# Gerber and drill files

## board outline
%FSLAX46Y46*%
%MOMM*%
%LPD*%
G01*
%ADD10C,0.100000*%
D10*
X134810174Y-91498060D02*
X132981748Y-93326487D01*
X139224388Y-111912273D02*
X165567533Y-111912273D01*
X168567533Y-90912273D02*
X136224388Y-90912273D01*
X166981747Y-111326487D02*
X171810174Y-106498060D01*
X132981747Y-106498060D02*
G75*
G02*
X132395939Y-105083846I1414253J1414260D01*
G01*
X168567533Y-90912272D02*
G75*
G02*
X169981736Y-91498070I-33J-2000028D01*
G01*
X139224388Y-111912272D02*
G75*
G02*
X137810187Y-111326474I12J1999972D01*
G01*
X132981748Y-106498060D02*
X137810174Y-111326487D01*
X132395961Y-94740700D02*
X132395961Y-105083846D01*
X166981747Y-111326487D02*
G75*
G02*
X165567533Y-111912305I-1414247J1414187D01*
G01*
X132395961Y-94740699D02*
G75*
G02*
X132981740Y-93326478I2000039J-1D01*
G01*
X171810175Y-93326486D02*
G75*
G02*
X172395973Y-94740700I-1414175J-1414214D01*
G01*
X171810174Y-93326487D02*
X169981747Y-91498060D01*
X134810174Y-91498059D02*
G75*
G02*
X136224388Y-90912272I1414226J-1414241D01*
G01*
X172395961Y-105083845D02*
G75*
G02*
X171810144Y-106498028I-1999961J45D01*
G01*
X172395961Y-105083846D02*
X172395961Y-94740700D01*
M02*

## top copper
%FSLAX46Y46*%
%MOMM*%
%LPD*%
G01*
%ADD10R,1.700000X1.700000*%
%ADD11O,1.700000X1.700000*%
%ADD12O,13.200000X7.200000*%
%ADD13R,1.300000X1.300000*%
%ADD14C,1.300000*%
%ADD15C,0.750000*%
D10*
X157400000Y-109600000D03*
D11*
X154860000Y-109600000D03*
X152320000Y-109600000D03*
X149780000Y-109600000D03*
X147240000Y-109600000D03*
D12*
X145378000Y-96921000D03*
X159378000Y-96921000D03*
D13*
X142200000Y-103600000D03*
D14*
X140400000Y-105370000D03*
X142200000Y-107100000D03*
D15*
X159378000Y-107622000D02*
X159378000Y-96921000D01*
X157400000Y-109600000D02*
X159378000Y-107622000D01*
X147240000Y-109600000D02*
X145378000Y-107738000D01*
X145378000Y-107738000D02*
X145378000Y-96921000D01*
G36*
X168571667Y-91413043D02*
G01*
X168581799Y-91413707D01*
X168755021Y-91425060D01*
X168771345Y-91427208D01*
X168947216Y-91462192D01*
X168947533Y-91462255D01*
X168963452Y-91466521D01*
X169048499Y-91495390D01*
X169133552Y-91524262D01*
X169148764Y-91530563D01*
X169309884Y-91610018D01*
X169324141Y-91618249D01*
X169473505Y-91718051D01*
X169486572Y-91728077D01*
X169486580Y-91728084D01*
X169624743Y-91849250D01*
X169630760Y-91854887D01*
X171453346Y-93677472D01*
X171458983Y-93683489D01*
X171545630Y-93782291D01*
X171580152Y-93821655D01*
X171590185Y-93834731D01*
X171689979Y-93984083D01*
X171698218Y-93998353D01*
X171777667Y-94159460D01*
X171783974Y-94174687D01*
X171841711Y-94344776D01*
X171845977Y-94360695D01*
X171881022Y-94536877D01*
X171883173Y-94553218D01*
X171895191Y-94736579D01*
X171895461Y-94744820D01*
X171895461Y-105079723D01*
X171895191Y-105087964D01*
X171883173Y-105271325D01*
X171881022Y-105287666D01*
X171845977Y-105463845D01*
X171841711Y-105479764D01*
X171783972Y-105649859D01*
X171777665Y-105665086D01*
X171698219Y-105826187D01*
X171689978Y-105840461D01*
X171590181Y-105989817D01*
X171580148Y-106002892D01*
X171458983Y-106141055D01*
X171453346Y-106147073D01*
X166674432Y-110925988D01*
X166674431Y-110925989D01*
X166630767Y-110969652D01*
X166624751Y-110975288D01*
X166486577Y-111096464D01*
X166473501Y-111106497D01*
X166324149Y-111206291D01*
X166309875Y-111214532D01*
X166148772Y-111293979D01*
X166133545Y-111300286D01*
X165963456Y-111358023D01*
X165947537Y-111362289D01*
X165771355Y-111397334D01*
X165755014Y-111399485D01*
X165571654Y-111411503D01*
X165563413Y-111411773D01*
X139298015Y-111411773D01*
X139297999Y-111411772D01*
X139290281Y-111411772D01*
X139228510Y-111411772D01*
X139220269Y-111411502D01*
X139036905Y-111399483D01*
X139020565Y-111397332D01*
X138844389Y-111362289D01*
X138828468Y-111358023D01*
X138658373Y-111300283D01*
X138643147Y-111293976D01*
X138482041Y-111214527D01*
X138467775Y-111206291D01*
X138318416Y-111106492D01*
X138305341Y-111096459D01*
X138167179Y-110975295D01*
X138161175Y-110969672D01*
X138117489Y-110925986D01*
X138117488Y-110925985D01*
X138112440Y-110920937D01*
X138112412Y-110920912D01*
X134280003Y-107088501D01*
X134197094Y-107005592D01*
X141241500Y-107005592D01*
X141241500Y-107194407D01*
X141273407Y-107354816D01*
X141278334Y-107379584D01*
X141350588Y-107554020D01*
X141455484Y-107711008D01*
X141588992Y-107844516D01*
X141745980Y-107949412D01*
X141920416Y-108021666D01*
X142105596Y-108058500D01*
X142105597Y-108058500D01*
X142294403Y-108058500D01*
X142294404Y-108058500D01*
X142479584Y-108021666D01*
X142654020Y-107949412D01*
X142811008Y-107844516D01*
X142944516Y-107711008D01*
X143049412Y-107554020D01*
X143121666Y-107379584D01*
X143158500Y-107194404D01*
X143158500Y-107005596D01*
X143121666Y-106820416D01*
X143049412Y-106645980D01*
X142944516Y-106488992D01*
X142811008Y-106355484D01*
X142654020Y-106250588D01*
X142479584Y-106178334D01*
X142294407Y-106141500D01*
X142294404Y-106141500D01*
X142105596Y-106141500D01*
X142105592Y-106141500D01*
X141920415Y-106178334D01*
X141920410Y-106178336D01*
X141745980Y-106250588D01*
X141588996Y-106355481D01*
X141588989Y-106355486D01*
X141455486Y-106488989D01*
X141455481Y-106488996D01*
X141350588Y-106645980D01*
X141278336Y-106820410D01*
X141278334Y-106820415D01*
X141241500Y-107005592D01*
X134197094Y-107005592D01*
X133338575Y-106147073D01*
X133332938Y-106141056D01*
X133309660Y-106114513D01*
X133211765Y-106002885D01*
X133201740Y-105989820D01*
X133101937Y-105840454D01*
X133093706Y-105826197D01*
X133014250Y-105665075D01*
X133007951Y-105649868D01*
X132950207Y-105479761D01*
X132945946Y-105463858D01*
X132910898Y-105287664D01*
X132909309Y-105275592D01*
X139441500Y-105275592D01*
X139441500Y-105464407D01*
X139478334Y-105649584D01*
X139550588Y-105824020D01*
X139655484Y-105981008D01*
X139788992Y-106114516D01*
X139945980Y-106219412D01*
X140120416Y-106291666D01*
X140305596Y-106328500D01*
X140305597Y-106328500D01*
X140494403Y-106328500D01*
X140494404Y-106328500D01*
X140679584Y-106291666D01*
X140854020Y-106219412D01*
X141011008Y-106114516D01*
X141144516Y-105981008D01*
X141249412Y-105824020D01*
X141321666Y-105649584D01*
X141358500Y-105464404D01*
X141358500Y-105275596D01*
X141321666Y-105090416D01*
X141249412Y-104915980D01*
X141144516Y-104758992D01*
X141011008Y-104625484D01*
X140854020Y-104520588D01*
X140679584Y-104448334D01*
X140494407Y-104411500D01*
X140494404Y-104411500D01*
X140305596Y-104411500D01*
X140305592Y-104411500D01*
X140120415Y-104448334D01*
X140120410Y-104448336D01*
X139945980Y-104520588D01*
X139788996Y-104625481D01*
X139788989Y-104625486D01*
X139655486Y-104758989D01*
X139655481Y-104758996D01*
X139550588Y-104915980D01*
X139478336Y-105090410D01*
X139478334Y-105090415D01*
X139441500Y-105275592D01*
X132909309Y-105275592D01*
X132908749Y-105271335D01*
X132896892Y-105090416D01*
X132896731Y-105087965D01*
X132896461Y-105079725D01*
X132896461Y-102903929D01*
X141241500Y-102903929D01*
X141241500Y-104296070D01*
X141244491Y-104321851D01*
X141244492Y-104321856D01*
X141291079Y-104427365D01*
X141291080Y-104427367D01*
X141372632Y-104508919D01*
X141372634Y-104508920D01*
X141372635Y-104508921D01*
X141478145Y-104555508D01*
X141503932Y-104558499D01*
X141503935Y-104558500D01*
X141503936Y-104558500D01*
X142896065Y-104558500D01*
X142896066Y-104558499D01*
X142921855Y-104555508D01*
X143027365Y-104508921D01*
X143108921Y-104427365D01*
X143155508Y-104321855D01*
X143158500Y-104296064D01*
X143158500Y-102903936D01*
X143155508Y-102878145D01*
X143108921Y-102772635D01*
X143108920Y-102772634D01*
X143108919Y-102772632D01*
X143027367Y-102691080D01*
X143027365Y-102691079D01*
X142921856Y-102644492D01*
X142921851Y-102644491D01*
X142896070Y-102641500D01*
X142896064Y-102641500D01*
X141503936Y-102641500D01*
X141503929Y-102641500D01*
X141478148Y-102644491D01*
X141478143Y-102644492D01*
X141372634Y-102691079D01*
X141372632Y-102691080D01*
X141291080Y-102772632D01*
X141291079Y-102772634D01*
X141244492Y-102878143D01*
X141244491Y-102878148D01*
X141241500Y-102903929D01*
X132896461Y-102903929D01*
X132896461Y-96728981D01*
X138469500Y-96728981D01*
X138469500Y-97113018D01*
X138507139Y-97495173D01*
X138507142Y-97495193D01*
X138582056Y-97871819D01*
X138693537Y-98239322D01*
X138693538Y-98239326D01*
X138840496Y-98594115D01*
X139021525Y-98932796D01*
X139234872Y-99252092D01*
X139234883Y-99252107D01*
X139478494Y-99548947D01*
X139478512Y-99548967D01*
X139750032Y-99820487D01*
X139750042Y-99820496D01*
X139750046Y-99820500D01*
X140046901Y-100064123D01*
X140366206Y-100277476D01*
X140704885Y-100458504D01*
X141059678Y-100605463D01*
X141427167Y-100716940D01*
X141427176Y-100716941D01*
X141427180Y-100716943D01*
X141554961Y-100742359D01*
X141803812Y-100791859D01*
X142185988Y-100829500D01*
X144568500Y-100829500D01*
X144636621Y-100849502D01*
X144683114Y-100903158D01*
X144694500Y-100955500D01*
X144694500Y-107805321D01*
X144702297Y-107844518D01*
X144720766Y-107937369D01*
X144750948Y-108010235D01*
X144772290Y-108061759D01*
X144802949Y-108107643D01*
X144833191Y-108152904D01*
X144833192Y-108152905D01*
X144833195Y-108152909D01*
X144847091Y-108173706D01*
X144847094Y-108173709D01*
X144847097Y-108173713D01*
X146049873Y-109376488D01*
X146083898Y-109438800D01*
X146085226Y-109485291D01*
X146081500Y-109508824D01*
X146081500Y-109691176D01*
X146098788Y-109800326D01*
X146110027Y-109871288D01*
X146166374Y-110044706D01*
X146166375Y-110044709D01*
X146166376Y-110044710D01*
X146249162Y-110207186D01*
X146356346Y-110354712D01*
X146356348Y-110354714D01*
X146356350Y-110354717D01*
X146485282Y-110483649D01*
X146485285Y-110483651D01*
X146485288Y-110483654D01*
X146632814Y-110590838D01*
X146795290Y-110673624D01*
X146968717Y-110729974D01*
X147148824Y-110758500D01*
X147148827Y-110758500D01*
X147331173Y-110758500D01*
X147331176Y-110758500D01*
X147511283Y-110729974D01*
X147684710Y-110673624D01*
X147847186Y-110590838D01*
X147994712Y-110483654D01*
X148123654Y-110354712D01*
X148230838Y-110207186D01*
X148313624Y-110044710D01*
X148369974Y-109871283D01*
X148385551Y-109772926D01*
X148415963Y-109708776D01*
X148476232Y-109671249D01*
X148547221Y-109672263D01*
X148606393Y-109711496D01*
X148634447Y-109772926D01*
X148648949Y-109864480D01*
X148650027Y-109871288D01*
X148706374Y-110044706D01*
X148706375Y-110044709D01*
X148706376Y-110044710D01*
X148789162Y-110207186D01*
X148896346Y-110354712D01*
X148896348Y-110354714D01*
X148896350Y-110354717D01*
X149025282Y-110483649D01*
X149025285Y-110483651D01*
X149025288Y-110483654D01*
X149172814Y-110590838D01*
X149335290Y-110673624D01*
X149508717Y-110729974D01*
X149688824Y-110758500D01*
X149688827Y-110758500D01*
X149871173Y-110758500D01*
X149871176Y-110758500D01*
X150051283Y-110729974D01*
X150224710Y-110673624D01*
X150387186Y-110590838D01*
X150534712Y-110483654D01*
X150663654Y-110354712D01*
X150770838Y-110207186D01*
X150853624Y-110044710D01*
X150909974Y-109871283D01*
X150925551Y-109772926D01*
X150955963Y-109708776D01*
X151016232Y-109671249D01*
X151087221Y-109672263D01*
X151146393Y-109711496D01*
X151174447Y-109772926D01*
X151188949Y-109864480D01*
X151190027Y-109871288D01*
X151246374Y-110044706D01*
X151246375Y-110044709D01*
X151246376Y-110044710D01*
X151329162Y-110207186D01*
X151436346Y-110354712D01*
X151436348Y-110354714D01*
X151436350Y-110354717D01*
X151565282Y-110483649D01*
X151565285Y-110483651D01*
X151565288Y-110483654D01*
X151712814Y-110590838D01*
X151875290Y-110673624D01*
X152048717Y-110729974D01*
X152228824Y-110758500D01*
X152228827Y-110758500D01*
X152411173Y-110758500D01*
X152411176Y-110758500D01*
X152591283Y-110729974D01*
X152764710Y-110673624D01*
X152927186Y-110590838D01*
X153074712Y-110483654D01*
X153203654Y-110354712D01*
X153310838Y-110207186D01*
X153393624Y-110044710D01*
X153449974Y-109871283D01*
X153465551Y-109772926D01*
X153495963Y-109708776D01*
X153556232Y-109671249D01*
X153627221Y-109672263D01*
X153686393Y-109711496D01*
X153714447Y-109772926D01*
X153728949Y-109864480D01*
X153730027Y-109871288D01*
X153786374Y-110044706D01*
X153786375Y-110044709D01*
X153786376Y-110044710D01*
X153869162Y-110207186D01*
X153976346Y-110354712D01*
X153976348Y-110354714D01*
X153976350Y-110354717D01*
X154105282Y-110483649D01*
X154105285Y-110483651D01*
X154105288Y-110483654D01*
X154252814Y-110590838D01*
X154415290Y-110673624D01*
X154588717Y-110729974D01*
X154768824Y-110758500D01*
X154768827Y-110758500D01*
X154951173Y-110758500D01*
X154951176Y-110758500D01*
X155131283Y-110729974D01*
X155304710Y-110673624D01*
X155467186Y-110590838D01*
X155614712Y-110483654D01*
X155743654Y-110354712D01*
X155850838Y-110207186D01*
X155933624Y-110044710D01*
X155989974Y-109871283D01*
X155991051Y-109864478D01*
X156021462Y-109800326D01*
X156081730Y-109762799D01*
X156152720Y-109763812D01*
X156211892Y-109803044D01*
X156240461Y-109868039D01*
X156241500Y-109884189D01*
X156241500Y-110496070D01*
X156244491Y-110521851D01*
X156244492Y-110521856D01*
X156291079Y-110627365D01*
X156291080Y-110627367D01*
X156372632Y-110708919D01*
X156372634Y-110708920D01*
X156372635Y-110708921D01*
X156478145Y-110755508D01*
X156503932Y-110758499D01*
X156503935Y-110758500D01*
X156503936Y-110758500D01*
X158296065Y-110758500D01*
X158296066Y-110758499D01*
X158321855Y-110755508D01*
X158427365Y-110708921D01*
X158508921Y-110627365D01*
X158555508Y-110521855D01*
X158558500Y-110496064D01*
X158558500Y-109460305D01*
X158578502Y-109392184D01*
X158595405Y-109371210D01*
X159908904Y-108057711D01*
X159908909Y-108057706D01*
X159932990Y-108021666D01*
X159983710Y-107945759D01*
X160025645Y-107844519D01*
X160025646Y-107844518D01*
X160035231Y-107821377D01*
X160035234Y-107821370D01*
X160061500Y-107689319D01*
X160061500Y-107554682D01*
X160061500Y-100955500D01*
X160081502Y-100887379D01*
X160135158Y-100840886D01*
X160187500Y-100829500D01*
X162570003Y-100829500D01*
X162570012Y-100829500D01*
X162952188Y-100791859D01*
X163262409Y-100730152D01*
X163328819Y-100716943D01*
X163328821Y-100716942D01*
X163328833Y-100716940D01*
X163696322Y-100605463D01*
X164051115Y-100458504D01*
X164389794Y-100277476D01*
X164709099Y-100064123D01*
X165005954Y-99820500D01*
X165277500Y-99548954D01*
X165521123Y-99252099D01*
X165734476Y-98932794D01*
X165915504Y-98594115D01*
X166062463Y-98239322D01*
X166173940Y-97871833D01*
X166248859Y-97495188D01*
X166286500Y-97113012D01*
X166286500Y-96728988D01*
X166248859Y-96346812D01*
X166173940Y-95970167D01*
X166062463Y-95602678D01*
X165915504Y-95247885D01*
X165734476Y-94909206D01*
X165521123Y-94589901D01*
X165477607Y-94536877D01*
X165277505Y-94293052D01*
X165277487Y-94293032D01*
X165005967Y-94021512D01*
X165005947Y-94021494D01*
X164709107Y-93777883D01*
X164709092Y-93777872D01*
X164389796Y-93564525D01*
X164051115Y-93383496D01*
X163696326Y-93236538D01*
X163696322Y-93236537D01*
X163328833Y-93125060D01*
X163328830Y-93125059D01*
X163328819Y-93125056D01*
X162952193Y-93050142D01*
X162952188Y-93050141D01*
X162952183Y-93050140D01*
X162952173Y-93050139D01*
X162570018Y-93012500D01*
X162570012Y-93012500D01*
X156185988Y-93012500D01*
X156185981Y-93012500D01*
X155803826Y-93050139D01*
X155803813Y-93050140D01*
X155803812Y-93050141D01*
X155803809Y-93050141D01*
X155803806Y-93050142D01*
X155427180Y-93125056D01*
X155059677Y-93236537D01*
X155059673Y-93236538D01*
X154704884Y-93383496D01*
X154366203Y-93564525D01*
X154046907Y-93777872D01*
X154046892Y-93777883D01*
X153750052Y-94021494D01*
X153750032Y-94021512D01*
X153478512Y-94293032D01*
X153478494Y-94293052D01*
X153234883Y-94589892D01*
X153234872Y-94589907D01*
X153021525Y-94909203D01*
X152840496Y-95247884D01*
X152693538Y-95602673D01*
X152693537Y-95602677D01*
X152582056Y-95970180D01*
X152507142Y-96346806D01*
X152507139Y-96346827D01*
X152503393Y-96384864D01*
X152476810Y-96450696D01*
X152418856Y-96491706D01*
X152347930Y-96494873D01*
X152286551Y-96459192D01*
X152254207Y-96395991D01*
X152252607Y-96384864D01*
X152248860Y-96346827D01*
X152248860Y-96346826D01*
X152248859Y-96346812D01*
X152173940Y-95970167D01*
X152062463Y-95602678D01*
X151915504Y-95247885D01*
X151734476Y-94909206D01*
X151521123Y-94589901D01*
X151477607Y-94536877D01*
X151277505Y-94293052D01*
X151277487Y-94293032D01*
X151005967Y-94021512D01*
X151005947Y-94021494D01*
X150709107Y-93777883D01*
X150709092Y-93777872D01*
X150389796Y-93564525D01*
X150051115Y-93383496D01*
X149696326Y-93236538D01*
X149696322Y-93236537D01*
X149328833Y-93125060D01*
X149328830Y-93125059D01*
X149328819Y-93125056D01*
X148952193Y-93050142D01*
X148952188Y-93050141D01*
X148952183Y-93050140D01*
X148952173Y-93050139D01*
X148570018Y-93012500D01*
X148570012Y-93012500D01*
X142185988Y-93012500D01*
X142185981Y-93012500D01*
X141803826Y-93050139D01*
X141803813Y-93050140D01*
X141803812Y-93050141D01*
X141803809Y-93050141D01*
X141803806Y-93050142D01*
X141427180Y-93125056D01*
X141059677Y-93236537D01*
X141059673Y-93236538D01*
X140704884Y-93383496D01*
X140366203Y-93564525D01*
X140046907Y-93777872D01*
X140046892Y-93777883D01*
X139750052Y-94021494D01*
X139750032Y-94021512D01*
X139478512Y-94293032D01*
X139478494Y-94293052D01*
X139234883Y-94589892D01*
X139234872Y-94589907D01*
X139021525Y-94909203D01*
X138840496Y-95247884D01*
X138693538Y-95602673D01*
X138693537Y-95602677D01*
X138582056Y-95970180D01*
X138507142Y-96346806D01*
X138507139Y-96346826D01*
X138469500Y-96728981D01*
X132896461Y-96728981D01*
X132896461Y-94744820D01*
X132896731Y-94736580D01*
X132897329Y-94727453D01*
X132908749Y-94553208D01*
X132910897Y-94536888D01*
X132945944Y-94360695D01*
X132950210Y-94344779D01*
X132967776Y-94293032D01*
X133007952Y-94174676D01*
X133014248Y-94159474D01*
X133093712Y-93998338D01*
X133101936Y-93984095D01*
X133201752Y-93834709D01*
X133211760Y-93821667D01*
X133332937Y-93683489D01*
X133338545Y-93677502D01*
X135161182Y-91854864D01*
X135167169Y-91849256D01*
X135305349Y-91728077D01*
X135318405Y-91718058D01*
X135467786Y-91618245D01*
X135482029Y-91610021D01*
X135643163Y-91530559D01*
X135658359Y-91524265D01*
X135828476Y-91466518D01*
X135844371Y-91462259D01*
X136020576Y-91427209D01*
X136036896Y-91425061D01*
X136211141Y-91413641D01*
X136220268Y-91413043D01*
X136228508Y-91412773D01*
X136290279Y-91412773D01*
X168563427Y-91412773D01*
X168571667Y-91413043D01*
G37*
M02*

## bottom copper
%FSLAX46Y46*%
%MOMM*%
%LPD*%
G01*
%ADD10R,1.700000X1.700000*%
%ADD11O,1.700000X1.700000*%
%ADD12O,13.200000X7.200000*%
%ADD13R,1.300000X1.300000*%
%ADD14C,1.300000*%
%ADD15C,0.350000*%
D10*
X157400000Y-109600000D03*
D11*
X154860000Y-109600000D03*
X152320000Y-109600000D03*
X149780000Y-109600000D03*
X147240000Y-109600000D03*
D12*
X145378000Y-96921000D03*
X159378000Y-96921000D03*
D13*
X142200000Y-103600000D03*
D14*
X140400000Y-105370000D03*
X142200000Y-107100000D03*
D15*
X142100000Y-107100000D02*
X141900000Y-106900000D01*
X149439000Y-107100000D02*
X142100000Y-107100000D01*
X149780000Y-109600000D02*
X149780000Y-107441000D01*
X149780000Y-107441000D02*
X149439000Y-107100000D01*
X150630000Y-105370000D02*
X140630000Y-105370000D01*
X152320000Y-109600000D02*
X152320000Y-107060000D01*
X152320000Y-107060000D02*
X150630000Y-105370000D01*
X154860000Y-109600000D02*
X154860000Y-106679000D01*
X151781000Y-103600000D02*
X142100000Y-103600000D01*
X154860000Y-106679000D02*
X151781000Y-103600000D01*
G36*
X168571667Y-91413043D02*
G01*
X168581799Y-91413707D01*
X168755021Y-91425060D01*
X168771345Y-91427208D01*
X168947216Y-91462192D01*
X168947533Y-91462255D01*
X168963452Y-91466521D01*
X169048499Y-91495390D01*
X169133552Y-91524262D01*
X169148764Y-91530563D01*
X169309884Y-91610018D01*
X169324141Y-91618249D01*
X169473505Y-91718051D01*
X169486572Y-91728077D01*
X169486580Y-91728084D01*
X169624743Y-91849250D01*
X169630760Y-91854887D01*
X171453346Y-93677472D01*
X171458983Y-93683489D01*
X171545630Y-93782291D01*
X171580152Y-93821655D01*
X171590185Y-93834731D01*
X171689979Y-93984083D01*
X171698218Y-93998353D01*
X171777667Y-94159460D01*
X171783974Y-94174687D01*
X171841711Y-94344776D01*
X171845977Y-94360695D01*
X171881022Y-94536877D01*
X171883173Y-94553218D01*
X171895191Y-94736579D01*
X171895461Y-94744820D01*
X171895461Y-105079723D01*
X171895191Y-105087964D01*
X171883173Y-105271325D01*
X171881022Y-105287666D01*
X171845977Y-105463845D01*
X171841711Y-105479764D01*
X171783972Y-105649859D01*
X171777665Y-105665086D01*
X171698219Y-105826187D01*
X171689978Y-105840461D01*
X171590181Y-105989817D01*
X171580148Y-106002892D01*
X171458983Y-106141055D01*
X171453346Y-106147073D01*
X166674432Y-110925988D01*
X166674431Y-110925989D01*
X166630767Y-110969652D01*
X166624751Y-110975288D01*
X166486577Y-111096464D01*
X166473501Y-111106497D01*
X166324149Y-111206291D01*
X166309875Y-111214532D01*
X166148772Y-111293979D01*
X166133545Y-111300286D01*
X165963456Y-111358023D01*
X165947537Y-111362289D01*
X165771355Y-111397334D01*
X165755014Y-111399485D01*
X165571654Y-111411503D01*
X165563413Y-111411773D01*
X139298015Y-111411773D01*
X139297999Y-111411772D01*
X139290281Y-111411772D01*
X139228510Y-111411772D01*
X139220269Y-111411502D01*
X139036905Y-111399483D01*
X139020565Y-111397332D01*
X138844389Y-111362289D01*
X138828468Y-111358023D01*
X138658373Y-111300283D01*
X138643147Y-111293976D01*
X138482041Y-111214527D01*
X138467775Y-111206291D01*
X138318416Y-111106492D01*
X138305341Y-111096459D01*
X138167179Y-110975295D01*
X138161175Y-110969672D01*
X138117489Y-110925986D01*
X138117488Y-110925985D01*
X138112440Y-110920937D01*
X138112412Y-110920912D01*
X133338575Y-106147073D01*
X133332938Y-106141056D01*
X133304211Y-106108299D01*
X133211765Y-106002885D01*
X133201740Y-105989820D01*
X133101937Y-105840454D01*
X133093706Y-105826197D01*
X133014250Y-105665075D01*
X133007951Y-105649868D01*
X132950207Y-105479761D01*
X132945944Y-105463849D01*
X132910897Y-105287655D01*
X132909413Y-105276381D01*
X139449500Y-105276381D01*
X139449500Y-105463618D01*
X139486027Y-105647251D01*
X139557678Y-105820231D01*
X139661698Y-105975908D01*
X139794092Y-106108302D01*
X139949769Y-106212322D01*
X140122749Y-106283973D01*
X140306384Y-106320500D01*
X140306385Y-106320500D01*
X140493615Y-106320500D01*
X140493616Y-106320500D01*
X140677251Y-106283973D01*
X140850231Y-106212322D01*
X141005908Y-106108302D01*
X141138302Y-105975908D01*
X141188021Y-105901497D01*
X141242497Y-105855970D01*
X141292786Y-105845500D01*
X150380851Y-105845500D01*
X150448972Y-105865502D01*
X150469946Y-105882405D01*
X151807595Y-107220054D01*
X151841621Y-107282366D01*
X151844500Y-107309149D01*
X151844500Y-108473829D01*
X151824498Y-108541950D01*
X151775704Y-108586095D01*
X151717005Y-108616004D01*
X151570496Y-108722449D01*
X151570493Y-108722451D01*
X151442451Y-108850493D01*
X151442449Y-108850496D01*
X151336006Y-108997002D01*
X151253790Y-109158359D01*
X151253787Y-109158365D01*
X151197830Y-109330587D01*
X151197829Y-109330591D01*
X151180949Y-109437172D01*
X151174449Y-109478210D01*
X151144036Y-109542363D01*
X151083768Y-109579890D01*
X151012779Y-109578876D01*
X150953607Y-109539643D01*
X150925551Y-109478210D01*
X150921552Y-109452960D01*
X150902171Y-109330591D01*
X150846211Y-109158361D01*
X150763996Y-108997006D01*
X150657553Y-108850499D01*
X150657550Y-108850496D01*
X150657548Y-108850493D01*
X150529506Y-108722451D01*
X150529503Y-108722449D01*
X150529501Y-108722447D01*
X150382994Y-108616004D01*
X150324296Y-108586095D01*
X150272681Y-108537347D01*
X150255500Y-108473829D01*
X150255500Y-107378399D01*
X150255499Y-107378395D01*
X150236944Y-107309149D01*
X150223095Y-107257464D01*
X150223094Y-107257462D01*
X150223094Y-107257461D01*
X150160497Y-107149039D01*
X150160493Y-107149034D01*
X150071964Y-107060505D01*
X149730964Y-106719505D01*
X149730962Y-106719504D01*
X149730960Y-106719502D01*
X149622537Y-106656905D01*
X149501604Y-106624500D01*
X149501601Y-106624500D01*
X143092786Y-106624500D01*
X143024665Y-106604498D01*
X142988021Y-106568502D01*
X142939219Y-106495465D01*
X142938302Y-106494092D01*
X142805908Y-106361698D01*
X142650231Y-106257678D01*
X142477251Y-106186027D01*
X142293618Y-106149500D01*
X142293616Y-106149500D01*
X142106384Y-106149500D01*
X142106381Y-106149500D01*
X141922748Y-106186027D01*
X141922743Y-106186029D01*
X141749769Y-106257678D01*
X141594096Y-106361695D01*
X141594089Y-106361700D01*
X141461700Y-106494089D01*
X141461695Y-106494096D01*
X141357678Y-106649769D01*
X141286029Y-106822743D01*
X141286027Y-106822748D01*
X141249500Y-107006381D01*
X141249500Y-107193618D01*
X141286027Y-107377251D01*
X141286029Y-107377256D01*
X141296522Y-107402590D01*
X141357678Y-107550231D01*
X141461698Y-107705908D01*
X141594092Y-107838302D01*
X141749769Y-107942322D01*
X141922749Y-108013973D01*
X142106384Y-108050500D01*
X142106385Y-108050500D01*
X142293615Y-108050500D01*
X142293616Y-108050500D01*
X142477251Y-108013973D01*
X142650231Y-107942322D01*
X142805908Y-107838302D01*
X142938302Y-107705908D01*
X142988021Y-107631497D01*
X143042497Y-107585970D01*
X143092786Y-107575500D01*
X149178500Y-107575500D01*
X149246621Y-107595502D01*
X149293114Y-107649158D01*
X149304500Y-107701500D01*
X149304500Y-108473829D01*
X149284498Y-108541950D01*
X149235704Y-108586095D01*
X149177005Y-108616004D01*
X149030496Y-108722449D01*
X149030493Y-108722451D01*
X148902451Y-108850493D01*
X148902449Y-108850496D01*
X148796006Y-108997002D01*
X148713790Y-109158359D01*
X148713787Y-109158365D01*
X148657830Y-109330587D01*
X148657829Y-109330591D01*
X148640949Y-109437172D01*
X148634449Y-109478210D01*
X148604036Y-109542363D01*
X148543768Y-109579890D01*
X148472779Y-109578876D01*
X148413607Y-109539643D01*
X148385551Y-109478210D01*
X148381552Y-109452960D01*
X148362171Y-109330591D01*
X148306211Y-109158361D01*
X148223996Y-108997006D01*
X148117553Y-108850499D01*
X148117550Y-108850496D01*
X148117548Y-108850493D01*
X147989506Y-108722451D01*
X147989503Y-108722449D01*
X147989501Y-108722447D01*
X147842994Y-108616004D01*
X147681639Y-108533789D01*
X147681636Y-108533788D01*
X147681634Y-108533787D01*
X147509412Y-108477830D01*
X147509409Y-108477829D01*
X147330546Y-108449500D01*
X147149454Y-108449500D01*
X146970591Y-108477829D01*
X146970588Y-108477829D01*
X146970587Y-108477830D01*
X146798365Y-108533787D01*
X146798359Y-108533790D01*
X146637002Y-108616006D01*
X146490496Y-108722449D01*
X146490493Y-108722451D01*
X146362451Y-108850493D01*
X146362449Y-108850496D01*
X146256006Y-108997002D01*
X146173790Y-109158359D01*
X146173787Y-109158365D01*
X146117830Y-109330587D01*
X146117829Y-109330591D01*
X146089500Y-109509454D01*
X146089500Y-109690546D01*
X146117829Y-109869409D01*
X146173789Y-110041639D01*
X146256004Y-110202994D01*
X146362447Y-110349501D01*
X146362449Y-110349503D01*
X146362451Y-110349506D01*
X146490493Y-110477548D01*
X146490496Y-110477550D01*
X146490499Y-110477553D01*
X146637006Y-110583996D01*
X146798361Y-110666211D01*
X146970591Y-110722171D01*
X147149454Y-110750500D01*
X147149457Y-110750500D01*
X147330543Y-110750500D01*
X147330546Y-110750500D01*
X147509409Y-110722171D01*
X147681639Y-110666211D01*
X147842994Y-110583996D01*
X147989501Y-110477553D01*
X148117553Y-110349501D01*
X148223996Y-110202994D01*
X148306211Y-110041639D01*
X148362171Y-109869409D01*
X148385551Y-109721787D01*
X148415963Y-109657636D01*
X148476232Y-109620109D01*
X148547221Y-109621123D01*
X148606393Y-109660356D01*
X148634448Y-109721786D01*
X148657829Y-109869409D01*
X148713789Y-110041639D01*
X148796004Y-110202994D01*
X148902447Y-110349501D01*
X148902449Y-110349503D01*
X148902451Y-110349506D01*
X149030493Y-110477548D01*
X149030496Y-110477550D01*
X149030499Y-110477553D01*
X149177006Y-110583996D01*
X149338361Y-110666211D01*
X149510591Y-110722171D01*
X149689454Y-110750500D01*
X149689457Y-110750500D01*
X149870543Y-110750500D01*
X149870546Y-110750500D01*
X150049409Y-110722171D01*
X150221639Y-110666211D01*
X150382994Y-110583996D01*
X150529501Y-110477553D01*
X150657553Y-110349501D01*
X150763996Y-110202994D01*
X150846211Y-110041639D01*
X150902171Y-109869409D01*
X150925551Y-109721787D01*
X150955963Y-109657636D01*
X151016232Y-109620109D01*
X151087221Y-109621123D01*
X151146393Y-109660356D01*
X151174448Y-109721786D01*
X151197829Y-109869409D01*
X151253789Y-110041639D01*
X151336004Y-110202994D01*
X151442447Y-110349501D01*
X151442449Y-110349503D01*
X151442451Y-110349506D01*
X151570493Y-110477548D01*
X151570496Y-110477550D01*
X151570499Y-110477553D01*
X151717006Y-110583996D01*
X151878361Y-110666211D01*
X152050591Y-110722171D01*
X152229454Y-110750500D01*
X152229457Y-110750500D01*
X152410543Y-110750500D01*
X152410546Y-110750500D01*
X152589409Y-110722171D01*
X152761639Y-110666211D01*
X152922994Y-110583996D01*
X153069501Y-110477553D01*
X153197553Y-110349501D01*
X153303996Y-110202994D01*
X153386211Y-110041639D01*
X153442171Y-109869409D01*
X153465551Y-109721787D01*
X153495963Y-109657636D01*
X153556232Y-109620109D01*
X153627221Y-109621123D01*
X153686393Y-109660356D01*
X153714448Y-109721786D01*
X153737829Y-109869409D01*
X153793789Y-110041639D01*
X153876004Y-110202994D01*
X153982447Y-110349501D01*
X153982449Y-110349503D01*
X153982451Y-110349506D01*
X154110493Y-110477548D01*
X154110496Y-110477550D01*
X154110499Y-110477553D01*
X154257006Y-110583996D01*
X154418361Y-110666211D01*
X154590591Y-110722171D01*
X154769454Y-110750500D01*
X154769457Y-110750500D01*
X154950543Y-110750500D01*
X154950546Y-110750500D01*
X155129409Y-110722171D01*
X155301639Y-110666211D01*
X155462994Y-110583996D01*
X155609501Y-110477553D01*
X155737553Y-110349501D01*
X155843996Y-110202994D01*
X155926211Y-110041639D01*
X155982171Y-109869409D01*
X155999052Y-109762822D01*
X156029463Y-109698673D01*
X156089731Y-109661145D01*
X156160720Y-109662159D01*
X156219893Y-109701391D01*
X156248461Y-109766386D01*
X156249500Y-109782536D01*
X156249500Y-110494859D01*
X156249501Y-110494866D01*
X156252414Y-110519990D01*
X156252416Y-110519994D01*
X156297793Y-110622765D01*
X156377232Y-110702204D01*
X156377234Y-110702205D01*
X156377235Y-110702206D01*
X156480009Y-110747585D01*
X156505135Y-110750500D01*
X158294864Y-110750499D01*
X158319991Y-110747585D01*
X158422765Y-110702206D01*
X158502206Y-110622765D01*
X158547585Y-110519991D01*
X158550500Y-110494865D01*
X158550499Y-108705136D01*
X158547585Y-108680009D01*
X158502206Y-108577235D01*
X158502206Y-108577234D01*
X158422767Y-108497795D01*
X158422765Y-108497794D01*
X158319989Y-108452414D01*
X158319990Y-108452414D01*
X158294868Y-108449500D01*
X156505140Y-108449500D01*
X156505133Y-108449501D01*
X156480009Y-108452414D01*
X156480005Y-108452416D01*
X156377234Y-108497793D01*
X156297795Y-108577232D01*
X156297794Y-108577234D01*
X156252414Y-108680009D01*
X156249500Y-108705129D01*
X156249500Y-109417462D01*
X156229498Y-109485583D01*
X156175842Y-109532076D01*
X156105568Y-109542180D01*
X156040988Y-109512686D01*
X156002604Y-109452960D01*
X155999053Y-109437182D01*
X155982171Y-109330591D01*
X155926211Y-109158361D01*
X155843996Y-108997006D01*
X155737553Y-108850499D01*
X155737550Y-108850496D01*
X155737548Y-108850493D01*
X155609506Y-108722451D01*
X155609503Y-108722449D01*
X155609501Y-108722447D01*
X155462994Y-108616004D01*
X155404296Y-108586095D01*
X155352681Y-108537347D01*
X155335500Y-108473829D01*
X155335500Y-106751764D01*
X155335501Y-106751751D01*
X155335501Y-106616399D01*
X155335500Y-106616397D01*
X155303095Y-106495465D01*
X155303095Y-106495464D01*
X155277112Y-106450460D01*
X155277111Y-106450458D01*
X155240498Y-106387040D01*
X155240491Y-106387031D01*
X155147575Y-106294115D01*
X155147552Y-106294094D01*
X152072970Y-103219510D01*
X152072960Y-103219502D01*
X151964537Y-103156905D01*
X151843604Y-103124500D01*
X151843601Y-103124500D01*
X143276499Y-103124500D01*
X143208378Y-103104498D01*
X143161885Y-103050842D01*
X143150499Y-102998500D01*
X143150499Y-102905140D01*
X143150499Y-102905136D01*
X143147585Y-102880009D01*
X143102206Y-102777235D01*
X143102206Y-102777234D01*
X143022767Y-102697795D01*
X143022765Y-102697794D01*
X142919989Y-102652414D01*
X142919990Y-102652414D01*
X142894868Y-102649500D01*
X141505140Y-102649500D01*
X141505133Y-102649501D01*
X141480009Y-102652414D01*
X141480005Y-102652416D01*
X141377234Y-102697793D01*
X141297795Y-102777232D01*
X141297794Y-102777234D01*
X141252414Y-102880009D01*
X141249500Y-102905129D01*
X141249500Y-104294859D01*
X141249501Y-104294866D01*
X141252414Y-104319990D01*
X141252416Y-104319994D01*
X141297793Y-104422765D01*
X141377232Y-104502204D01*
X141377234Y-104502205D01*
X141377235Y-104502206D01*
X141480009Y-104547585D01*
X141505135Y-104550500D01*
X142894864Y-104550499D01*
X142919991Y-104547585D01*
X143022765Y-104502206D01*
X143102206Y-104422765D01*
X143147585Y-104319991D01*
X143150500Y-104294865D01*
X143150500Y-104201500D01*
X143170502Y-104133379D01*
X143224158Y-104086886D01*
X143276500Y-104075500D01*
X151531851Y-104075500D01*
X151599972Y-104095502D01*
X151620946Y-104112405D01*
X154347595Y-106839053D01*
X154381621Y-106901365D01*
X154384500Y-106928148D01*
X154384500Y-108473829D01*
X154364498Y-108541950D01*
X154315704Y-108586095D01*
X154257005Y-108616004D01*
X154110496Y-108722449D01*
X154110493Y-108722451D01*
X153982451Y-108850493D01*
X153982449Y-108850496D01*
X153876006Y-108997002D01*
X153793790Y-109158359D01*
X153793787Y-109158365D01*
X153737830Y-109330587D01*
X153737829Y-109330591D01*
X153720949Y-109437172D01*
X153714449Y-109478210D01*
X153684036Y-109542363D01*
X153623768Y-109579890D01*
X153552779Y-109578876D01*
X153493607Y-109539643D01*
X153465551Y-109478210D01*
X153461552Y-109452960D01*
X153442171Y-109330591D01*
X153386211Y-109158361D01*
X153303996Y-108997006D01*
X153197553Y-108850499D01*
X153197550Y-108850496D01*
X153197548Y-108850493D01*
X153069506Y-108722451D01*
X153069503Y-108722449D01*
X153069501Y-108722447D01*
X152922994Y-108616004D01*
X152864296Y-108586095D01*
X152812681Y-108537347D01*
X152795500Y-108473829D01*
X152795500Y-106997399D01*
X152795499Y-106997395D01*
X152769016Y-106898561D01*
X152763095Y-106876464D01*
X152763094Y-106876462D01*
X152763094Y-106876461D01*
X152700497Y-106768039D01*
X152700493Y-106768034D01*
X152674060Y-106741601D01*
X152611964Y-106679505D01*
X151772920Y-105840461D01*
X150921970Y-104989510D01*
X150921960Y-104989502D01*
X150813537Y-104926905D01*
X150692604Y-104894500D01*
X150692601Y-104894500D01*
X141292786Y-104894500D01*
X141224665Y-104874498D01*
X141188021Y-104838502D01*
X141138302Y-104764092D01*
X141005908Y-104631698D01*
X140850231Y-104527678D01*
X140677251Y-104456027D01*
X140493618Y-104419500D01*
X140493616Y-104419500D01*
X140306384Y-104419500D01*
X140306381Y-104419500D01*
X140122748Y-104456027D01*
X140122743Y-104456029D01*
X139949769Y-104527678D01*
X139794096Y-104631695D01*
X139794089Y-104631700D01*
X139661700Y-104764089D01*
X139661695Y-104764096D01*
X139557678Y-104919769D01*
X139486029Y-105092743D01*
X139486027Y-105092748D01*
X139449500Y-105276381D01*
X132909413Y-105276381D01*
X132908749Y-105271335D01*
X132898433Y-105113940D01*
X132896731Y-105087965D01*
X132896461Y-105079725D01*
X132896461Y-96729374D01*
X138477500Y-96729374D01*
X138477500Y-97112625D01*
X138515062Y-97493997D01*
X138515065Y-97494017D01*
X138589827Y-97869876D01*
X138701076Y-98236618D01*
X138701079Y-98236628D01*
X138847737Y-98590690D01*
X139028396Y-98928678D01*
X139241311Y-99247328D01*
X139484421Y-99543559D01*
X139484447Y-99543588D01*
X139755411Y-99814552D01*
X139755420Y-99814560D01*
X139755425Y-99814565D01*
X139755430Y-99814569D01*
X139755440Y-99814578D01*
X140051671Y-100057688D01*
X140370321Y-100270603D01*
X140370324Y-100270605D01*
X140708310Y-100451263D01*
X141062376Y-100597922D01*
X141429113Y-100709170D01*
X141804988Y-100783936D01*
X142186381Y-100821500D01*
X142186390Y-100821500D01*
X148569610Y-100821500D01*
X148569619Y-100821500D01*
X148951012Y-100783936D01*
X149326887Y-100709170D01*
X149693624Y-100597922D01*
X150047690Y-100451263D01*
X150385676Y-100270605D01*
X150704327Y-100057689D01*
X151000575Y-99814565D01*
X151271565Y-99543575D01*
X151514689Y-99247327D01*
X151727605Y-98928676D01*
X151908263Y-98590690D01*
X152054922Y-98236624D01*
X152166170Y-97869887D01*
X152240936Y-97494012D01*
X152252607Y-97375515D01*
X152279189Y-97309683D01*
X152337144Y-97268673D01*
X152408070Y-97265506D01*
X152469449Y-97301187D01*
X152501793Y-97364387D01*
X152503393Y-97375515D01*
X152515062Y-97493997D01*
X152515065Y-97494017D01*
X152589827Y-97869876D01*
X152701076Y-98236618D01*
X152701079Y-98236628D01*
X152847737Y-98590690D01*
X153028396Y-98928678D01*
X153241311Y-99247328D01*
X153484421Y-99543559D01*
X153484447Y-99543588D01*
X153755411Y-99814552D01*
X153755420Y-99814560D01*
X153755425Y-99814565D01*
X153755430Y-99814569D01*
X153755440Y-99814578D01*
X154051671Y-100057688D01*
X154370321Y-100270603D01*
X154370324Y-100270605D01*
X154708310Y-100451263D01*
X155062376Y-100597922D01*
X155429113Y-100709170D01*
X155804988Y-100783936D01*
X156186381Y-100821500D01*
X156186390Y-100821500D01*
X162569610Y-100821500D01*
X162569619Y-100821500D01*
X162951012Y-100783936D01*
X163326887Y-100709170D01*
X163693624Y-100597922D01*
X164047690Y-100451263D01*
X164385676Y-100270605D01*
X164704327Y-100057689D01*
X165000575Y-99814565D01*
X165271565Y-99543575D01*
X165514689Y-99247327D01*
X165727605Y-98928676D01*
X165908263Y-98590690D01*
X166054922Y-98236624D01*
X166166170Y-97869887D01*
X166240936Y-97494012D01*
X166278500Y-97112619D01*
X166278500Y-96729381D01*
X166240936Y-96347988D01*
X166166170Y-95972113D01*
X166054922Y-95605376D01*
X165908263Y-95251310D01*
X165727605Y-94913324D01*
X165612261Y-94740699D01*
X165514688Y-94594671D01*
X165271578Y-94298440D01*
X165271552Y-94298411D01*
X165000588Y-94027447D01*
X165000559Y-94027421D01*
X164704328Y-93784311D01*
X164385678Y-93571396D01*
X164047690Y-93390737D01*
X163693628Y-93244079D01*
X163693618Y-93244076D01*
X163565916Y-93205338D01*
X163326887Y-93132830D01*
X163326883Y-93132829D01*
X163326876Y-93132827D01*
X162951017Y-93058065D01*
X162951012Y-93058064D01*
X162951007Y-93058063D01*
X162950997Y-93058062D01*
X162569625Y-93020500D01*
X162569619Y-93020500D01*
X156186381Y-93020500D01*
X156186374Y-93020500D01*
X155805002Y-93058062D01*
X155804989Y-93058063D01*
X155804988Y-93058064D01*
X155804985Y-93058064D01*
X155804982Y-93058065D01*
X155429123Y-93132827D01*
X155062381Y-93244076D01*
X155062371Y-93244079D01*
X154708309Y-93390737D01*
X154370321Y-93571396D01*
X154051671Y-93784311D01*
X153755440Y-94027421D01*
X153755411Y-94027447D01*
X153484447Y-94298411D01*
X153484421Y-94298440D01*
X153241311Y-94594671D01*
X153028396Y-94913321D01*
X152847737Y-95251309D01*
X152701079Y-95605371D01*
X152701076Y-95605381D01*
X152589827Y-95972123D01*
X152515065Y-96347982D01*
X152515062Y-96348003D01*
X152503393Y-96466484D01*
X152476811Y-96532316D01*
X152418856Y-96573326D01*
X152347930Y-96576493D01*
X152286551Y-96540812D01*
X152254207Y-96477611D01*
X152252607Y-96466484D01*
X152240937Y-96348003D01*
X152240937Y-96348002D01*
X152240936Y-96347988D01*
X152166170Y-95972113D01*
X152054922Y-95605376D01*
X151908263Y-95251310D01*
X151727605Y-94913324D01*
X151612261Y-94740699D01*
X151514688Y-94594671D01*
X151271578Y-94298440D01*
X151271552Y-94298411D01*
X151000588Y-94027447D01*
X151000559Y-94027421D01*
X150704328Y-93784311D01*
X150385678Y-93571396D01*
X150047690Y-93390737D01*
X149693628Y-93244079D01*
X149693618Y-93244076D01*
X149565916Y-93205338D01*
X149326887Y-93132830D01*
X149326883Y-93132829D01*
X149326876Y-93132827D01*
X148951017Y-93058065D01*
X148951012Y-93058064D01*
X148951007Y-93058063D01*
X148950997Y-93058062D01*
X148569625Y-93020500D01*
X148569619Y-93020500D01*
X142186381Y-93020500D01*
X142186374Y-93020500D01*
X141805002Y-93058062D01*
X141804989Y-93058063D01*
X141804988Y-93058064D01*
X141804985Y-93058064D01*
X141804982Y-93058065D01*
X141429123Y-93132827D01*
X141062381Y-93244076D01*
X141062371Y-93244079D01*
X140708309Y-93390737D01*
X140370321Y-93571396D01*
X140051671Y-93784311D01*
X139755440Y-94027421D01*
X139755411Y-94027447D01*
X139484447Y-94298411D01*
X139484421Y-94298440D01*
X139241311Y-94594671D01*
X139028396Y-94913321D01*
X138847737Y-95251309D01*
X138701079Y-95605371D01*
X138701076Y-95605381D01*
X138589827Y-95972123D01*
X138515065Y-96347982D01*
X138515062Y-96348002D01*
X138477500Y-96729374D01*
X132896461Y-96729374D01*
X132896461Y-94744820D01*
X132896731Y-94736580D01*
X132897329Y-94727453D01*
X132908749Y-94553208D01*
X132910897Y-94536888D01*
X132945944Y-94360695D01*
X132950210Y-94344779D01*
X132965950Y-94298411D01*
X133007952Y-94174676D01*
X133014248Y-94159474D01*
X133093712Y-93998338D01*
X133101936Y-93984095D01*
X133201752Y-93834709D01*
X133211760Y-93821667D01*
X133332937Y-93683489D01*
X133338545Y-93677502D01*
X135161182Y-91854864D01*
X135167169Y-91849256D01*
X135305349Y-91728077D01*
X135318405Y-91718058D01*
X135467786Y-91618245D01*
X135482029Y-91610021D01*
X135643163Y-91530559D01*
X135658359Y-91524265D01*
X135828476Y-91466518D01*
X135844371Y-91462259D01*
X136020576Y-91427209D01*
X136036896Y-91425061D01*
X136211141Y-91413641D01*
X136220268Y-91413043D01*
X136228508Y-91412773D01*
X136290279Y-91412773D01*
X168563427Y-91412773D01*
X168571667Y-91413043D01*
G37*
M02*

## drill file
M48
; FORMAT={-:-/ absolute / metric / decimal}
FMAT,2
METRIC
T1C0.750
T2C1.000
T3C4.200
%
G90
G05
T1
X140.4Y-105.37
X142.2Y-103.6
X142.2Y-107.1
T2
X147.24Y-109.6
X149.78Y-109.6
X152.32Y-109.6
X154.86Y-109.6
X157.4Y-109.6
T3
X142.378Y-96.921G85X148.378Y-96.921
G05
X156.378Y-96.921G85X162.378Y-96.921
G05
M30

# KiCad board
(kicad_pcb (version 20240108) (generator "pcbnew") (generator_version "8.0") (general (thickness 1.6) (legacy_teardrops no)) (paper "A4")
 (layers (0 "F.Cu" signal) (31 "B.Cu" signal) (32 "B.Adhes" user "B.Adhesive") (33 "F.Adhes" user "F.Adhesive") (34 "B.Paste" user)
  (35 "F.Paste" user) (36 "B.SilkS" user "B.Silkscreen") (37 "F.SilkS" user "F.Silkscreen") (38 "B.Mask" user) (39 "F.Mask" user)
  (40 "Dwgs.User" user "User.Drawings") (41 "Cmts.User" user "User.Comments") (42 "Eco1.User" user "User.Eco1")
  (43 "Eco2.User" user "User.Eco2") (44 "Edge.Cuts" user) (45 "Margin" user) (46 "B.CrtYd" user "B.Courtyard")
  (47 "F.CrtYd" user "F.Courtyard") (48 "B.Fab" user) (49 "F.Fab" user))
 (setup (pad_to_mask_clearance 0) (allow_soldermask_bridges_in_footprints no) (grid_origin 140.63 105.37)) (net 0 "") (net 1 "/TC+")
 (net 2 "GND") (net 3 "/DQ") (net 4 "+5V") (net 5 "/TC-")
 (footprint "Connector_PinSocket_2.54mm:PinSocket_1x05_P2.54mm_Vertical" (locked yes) (layer "F.Cu") (at 157.4 109.6 -90)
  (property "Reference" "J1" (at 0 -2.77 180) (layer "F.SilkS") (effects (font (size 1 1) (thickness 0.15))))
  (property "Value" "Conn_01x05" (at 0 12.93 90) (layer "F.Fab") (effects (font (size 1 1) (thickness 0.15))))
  (pad "1" thru_hole rect (at 0 0 270) (size 1.7 1.7) (drill 1) (layers "*.Cu" "*.Mask") (remove_unused_layers no) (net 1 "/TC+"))
  (pad "2" thru_hole oval (at 0 2.54 270) (size 1.7 1.7) (drill 1) (layers "*.Cu" "*.Mask") (remove_unused_layers no) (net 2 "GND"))
  (pad "3" thru_hole oval (at 0 5.08 270) (size 1.7 1.7) (drill 1) (layers "*.Cu" "*.Mask") (remove_unused_layers no) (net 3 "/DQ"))
  (pad "4" thru_hole oval (at 0 7.62 270) (size 1.7 1.7) (drill 1) (layers "*.Cu" "*.Mask") (remove_unused_layers no) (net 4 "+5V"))
  (pad "5" thru_hole oval (at 0 10.16 270) (size 1.7 1.7) (drill 1) (layers "*.Cu" "*.Mask") (remove_unused_layers no) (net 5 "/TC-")))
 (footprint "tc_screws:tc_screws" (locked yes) (layer "F.Cu") (at 152.378 96.921)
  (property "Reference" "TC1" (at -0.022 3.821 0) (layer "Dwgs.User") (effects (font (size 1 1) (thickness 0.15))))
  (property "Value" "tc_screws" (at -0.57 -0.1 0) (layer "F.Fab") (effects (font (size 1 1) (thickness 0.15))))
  (pad "1" thru_hole oval (at -7 0) (size 13.2 7.2) (drill oval 10.2 4.2) (layers "*.Cu" "*.Mask") (remove_unused_layers no) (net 5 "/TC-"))
  (pad "2" thru_hole oval (at 7 0) (size 13.2 7.2) (drill oval 10.2 4.2) (layers "*.Cu" "*.Mask") (remove_unused_layers no) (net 1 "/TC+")))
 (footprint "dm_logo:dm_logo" (layer "F.Cu") (at 166.395961 103.912273)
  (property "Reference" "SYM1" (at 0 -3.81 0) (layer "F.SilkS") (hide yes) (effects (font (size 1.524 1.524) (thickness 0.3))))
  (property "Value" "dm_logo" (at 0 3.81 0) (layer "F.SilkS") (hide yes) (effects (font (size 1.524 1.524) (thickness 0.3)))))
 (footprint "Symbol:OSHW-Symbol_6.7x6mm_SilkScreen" (layer "F.Cu") (at 136.395961 103.412273)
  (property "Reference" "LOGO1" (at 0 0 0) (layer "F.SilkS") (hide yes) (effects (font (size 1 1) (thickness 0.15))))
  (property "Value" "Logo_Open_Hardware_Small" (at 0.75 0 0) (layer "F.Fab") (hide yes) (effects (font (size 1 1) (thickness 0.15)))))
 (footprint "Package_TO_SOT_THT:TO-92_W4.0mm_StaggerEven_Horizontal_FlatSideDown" (layer "B.Cu") (at 141.9 104.1 -90)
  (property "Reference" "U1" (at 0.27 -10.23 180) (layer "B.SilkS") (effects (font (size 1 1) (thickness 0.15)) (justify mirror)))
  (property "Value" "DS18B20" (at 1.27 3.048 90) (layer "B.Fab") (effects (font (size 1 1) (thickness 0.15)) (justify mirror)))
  (pad "1" thru_hole rect (at -0.5 -0.3 180) (size 1.3 1.3) (drill 0.75) (layers "*.Cu" "*.Mask") (remove_unused_layers no) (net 2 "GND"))
  (pad "2" thru_hole circle (at 1.27 1.5 180) (size 1.3 1.3) (drill 0.75) (layers "*.Cu" "*.Mask") (remove_unused_layers no) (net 3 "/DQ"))
  (pad "3" thru_hole circle (at 3 -0.3 180) (size 1.3 1.3) (drill 0.75) (layers "*.Cu" "*.Mask") (remove_unused_layers no) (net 4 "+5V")))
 (gr_line (start 134.810174 91.49806) (end 132.981748 93.326487) (stroke (width 0.1) (type solid)) (layer "Edge.Cuts"))
 (gr_line (start 139.224388 111.912273) (end 165.567533 111.912273) (stroke (width 0.1) (type solid)) (layer "Edge.Cuts"))
 (gr_line (start 168.567533 90.912273) (end 136.224388 90.912273) (stroke (width 0.1) (type solid)) (layer "Edge.Cuts"))
 (gr_line (start 166.981747 111.326487) (end 171.810174 106.49806) (stroke (width 0.1) (type solid)) (layer "Edge.Cuts"))
 (gr_arc (start 132.981747 106.49806) (mid 132.548201 105.849213) (end 132.395961 105.083846) (stroke (width 0.1) (type solid))
  (layer "Edge.Cuts"))
 (gr_arc (start 168.567533 90.912272) (mid 169.3329 91.064513) (end 169.981747 91.498059) (stroke (width 0.1) (type solid))
  (layer "Edge.Cuts"))
 (gr_arc (start 139.224388 111.912272) (mid 138.459022 111.760031) (end 137.810175 111.326486) (stroke (width 0.1) (type solid))
  (layer "Edge.Cuts"))
 (gr_line (start 132.981748 106.49806) (end 137.810174 111.326487) (stroke (width 0.1) (type solid)) (layer "Edge.Cuts"))
 (gr_line (start 132.395961 94.7407) (end 132.395961 105.083846) (stroke (width 0.1) (type solid)) (layer "Edge.Cuts"))
 (gr_arc (start 166.981747 111.326487) (mid 166.3329 111.760033) (end 165.567533 111.912273) (stroke (width 0.1) (type solid))
  (layer "Edge.Cuts"))
 (gr_arc (start 132.395961 94.740699) (mid 132.548202 93.975332) (end 132.981748 93.326486) (stroke (width 0.1) (type solid))
  (layer "Edge.Cuts"))
 (gr_arc (start 171.810175 93.326486) (mid 172.243721 93.975333) (end 172.395961 94.7407) (stroke (width 0.1) (type solid))
  (layer "Edge.Cuts"))
 (gr_line (start 171.810174 93.326487) (end 169.981747 91.49806) (stroke (width 0.1) (type solid)) (layer "Edge.Cuts"))
 (gr_arc (start 134.810174 91.498059) (mid 135.459021 91.064513) (end 136.224388 90.912273) (stroke (width 0.1) (type solid))
  (layer "Edge.Cuts"))
 (gr_arc (start 172.395961 105.083845) (mid 172.24372 105.849212) (end 171.810175 106.498059) (stroke (width 0.1) (type solid))
  (layer "Edge.Cuts"))
 (gr_line (start 172.395961 105.083846) (end 172.395961 94.7407) (stroke (width 0.1) (type solid)) (layer "Edge.Cuts"))
 (segment (start 159.378 107.622) (end 159.378 96.921) (width 0.75) (layer "F.Cu") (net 1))
 (segment (start 157.4 109.6) (end 159.378 107.622) (width 0.75) (layer "F.Cu") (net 1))
 (segment (start 142.1 107.1) (end 141.9 106.9) (width 0.35) (layer "B.Cu") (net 4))
 (segment (start 149.439 107.1) (end 142.1 107.1) (width 0.35) (layer "B.Cu") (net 4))
 (segment (start 149.78 109.6) (end 149.78 107.441) (width 0.35) (layer "B.Cu") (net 4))
 (segment (start 149.78 107.441) (end 149.439 107.1) (width 0.35) (layer "B.Cu") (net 4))
 (segment (start 150.63 105.37) (end 140.63 105.37) (width 0.35) (layer "B.Cu") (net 3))
 (segment (start 152.32 109.6) (end 152.32 107.06) (width 0.35) (layer "B.Cu") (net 3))
 (segment (start 152.32 107.06) (end 150.63 105.37) (width 0.35) (layer "B.Cu") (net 3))
 (segment (start 154.86 109.6) (end 154.86 106.679) (width 0.35) (layer "B.Cu") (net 2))
 (segment (start 151.781 103.6) (end 142.1 103.6) (width 0.35) (layer "B.Cu") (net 2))
 (segment (start 154.86 106.679) (end 151.781 103.6) (width 0.35) (layer "B.Cu") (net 2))
 (segment (start 147.24 109.6) (end 145.378 107.738) (width 0.75) (layer "F.Cu") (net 5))
 (segment (start 145.378 107.738) (end 145.378 96.921) (width 0.75) (layer "F.Cu") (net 5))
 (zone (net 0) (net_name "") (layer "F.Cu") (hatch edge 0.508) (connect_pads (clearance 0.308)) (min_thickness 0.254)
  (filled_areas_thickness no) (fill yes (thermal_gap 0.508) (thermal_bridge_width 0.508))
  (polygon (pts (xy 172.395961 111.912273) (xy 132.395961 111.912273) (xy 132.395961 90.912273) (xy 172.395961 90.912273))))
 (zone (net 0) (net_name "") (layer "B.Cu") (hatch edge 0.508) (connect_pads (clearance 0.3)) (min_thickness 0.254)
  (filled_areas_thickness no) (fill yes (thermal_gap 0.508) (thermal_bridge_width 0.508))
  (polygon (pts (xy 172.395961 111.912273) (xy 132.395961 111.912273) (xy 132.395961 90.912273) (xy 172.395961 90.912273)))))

